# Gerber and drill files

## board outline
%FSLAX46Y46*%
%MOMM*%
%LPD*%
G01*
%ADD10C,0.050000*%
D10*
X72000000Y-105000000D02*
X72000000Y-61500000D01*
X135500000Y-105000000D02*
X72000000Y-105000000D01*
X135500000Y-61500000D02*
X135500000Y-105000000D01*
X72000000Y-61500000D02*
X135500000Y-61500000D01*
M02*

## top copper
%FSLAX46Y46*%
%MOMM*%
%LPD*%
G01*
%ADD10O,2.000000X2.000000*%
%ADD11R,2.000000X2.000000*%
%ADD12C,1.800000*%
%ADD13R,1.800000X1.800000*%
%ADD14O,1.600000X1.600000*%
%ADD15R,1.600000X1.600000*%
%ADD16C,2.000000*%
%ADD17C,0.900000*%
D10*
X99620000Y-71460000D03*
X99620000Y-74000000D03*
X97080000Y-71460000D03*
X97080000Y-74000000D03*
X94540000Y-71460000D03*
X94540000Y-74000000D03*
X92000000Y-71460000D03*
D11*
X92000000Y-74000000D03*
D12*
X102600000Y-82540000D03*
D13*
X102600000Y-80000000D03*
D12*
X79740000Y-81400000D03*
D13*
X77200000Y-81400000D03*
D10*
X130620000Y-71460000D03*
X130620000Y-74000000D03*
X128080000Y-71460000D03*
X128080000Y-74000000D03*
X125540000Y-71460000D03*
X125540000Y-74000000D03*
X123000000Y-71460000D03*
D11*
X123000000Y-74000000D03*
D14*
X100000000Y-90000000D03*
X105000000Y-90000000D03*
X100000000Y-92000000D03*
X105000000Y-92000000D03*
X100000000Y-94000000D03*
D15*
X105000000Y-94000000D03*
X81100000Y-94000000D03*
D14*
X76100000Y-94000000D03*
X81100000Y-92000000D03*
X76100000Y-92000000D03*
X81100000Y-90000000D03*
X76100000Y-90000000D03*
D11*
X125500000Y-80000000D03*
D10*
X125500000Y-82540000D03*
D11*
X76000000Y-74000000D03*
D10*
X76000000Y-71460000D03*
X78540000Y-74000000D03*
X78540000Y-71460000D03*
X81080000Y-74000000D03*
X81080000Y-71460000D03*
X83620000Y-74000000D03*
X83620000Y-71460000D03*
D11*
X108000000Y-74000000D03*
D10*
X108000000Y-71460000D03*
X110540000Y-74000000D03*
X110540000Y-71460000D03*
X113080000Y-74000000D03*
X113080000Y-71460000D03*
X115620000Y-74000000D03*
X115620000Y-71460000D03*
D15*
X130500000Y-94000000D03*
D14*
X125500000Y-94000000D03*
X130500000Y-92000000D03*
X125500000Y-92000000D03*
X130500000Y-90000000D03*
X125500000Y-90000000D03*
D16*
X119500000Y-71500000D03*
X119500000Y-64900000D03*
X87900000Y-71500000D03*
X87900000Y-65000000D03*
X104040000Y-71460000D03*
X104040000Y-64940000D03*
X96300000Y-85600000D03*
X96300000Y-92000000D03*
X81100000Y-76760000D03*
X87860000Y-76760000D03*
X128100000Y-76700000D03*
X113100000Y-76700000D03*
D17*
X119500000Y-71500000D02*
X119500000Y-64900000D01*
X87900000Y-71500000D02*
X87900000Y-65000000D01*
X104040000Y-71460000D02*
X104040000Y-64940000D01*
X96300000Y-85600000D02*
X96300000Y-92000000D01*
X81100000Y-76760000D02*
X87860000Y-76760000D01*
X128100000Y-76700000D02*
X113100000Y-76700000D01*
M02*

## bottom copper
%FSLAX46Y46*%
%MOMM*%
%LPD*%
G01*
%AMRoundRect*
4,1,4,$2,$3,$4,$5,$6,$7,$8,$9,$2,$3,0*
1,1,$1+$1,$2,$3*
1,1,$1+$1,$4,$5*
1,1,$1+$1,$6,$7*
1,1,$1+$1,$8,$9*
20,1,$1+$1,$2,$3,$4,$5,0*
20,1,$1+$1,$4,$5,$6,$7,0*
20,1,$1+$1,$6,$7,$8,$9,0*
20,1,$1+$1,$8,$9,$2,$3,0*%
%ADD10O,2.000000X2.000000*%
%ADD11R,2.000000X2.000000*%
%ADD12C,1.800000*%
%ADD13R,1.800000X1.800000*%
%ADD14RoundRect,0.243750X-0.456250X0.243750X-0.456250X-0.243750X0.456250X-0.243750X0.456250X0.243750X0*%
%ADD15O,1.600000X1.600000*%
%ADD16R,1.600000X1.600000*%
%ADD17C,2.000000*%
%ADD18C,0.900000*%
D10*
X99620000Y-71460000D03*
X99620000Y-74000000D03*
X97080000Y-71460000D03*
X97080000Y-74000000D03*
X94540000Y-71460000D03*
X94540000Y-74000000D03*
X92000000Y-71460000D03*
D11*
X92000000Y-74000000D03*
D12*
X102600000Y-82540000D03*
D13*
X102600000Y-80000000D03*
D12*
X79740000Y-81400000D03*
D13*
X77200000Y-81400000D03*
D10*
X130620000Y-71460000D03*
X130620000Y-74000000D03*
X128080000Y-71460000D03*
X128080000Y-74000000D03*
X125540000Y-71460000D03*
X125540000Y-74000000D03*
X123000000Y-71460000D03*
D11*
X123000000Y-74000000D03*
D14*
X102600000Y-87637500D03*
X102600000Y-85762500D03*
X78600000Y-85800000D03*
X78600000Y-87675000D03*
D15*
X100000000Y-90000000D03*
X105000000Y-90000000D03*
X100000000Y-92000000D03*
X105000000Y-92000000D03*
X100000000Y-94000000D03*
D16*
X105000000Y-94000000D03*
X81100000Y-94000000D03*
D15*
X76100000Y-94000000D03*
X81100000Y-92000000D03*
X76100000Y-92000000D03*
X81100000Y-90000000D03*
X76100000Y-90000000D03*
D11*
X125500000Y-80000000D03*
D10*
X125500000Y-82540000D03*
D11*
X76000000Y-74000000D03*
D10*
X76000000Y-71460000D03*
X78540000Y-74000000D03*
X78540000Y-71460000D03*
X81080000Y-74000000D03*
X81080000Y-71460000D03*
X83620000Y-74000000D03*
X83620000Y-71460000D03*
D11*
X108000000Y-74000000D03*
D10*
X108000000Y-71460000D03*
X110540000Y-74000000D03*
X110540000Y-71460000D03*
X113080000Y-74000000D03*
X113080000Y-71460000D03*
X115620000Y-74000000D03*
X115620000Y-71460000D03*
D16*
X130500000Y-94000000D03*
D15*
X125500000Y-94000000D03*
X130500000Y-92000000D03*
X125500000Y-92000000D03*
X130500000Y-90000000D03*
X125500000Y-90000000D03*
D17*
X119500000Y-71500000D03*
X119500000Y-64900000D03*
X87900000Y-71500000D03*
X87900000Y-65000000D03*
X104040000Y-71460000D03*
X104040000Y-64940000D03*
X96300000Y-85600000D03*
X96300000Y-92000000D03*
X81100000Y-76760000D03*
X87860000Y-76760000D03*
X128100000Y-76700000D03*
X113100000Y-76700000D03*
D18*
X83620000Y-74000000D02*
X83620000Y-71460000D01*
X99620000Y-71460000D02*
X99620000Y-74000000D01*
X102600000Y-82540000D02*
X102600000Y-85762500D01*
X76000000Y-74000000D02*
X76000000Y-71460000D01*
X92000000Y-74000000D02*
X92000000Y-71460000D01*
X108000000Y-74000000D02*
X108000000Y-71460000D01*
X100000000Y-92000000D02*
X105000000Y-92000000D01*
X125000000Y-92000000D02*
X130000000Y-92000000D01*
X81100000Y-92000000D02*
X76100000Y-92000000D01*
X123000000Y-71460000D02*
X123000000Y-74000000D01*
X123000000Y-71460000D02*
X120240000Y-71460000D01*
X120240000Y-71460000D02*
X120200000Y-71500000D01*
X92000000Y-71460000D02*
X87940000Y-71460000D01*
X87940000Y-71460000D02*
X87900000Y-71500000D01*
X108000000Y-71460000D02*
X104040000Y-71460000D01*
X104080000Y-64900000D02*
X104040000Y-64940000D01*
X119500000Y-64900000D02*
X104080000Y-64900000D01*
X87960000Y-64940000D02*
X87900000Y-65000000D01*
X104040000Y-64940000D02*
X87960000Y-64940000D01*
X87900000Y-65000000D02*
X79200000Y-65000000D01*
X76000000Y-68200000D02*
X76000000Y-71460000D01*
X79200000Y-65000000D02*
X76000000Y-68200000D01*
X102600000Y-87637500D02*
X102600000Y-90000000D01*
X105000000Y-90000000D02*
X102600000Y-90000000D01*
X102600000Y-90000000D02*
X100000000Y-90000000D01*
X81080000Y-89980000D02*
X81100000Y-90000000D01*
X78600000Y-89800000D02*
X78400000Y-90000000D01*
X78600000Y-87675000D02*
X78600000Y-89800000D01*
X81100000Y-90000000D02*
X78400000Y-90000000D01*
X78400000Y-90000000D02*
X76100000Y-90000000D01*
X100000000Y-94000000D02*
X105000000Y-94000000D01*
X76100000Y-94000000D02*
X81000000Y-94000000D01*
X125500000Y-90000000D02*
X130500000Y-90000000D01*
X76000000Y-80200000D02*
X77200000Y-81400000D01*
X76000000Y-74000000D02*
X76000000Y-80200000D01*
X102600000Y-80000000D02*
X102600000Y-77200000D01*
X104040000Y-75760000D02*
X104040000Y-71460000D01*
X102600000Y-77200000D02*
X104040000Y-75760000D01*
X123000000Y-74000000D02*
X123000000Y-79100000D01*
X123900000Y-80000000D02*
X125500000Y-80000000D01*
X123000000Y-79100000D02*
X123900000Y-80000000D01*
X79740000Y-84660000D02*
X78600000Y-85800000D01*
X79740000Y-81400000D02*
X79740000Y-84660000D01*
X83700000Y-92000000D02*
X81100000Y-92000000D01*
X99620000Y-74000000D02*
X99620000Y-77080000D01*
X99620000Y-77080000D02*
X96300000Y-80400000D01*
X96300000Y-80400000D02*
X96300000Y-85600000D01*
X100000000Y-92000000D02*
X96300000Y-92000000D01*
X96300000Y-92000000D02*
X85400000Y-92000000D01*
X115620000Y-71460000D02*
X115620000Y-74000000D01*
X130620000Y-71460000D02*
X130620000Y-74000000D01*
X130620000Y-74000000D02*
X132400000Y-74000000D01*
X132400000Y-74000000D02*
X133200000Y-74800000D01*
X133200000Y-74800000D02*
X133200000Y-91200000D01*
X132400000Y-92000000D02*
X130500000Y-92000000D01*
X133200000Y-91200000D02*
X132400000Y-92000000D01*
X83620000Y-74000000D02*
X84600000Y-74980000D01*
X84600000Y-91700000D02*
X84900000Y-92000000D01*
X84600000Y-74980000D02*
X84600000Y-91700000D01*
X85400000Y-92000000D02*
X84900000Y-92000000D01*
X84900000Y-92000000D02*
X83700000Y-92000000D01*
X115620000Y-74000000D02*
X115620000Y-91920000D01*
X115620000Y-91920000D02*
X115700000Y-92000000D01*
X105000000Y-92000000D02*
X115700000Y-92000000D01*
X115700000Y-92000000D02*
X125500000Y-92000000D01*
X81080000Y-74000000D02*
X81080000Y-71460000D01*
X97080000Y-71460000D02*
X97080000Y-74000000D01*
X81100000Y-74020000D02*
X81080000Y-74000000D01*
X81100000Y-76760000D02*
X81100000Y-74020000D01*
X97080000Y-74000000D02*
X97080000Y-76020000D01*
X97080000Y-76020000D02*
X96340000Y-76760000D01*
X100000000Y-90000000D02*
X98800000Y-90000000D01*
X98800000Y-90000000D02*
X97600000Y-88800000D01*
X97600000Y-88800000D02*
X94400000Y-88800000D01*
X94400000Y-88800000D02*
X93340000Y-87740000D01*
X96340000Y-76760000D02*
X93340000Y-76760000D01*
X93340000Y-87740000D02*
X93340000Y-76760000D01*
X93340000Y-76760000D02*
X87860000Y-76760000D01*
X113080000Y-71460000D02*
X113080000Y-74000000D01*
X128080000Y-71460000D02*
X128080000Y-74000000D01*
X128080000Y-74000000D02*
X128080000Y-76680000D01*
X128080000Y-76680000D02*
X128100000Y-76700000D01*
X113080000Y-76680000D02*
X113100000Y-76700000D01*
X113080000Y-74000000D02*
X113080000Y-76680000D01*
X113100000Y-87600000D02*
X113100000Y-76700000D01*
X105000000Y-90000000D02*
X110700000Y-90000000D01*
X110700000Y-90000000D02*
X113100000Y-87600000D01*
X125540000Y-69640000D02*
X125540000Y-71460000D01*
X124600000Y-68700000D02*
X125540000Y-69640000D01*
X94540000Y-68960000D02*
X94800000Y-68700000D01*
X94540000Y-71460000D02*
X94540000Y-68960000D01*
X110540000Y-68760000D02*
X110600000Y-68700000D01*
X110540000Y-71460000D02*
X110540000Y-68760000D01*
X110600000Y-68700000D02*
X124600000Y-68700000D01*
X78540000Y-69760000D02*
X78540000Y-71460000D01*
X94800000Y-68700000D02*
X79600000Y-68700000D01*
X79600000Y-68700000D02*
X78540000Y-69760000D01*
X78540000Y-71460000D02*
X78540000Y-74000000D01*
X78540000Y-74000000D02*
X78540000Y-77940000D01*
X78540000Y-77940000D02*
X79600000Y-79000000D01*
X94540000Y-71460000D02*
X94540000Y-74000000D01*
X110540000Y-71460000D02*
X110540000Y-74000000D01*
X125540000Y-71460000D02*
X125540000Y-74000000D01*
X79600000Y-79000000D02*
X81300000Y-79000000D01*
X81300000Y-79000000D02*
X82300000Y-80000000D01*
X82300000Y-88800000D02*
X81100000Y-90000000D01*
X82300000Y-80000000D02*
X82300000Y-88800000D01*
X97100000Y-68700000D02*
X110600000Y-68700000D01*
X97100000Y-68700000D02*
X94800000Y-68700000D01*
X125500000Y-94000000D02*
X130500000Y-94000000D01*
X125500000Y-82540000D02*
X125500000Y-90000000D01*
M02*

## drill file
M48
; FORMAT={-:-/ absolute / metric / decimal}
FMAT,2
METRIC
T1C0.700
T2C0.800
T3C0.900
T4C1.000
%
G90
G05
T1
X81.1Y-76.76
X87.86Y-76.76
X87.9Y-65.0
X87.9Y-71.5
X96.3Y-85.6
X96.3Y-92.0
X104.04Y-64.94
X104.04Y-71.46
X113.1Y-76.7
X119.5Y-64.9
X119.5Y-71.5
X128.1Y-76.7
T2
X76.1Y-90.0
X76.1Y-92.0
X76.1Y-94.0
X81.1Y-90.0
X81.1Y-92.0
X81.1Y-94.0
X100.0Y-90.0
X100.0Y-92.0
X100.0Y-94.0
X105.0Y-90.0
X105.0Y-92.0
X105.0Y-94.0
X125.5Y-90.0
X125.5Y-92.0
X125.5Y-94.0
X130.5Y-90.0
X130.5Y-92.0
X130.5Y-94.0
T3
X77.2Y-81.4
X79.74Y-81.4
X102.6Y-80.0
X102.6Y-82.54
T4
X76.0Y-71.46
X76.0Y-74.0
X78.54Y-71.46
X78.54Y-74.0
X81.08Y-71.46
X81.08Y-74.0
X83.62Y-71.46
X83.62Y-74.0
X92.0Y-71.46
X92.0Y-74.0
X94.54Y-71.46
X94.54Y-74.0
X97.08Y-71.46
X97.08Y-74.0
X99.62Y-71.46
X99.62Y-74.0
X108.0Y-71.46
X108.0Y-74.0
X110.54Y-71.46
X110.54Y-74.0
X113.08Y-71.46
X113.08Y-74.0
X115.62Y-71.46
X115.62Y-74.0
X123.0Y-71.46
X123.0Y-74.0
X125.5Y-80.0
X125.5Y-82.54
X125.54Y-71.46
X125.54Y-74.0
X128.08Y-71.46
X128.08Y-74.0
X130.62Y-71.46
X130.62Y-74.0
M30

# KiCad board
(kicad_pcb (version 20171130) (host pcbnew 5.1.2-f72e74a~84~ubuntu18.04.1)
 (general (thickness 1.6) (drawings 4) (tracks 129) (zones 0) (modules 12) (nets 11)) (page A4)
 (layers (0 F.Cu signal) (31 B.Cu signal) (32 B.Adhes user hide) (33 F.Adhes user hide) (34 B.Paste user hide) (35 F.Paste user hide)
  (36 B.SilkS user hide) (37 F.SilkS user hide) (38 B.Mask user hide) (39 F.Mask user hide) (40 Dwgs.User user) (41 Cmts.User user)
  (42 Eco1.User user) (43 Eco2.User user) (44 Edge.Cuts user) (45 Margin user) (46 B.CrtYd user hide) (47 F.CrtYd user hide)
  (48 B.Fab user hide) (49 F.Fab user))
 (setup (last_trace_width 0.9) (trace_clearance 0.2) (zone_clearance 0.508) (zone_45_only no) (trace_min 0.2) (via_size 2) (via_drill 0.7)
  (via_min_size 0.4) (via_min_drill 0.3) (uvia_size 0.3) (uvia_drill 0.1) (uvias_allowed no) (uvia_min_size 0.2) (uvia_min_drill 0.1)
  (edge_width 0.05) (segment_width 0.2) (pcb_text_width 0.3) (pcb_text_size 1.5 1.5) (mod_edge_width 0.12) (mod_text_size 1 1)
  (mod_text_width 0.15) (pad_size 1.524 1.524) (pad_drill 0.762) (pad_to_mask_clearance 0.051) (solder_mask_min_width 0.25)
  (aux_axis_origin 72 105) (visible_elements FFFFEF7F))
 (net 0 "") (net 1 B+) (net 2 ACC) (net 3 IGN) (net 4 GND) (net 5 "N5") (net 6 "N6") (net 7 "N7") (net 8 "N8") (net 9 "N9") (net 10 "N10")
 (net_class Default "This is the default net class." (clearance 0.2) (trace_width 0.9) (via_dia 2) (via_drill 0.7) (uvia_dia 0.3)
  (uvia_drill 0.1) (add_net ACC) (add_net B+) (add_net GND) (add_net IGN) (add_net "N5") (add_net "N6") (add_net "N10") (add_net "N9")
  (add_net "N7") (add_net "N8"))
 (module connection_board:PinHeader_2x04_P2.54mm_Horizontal (layer F.Cu) (at 92 74 90)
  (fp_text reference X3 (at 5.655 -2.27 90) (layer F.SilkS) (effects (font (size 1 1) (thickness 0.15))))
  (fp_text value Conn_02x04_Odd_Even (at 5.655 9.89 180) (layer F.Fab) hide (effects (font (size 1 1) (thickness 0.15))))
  (pad 8 thru_hole oval (at 2.54 7.62 90) (size 2 2) (drill 1) (layers *.Cu *.Mask) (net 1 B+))
  (pad 7 thru_hole oval (at 0 7.62 90) (size 2 2) (drill 1) (layers *.Cu *.Mask) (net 1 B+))
  (pad 6 thru_hole oval (at 2.54 5.08 90) (size 2 2) (drill 1) (layers *.Cu *.Mask) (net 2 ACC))
  (pad 5 thru_hole oval (at 0 5.08 90) (size 2 2) (drill 1) (layers *.Cu *.Mask) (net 2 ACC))
  (pad 4 thru_hole oval (at 2.54 2.54 90) (size 2 2) (drill 1) (layers *.Cu *.Mask) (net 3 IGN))
  (pad 3 thru_hole oval (at 0 2.54 90) (size 2 2) (drill 1) (layers *.Cu *.Mask) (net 3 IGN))
  (pad 2 thru_hole oval (at 2.54 0 90) (size 2 2) (drill 1) (layers *.Cu *.Mask) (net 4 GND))
  (pad 1 thru_hole rect (at 0 0 90) (size 2 2) (drill 1) (layers *.Cu *.Mask) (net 4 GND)))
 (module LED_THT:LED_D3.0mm (layer F.Cu) (at 102.6 80 270)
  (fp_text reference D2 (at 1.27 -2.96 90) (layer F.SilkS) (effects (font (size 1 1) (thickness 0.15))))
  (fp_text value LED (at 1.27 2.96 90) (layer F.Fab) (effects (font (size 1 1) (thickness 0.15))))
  (pad 2 thru_hole circle (at 2.54 0 270) (size 1.8 1.8) (drill 0.9) (layers *.Cu *.Mask) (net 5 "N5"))
  (pad 1 thru_hole rect (at 0 0 270) (size 1.8 1.8) (drill 0.9) (layers *.Cu *.Mask) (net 4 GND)))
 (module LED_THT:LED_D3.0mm (layer F.Cu) (at 77.2 81.4)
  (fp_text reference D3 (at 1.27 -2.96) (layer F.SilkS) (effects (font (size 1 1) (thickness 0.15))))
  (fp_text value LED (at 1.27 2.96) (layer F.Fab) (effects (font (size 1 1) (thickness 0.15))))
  (pad 2 thru_hole circle (at 2.54 0) (size 1.8 1.8) (drill 0.9) (layers *.Cu *.Mask) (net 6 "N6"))
  (pad 1 thru_hole rect (at 0 0) (size 1.8 1.8) (drill 0.9) (layers *.Cu *.Mask) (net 4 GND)))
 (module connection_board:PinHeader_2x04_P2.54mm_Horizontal (layer F.Cu) (at 123 74 90)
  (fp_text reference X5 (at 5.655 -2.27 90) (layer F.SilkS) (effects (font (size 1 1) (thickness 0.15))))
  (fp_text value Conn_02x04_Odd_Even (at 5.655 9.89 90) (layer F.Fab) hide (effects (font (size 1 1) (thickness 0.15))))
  (pad 8 thru_hole oval (at 2.54 7.62 90) (size 2 2) (drill 1) (layers *.Cu *.Mask) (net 1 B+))
  (pad 7 thru_hole oval (at 0 7.62 90) (size 2 2) (drill 1) (layers *.Cu *.Mask) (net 1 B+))
  (pad 6 thru_hole oval (at 2.54 5.08 90) (size 2 2) (drill 1) (layers *.Cu *.Mask) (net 2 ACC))
  (pad 5 thru_hole oval (at 0 5.08 90) (size 2 2) (drill 1) (layers *.Cu *.Mask) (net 2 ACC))
  (pad 4 thru_hole oval (at 2.54 2.54 90) (size 2 2) (drill 1) (layers *.Cu *.Mask) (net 3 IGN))
  (pad 3 thru_hole oval (at 0 2.54 90) (size 2 2) (drill 1) (layers *.Cu *.Mask) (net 3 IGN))
  (pad 2 thru_hole oval (at 2.54 0 90) (size 2 2) (drill 1) (layers *.Cu *.Mask) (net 4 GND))
  (pad 1 thru_hole rect (at 0 0 90) (size 2 2) (drill 1) (layers *.Cu *.Mask) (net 4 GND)))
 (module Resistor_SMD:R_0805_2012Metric (layer B.Cu) (at 102.6 86.7 270)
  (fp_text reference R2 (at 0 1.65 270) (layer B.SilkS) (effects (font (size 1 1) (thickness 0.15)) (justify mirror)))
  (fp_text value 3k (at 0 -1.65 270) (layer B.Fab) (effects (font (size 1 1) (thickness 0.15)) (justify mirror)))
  (pad 2 smd roundrect (at 0.9375 0 270) (size 0.975 1.4) (layers B.Cu B.Paste B.Mask) (roundrect_rratio 0.25) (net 2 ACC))
  (pad 1 smd roundrect (at -0.9375 0 270) (size 0.975 1.4) (layers B.Cu B.Paste B.Mask) (roundrect_rratio 0.25) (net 5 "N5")))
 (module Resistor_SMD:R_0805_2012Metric (layer B.Cu) (at 78.6 86.7375 270)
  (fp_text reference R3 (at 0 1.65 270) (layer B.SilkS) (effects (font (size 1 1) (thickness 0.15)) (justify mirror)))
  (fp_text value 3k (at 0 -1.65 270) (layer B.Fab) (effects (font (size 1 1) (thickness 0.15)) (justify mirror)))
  (pad 1 smd roundrect (at -0.9375 0 270) (size 0.975 1.4) (layers B.Cu B.Paste B.Mask) (roundrect_rratio 0.25) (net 6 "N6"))
  (pad 2 smd roundrect (at 0.9375 0 270) (size 0.975 1.4) (layers B.Cu B.Paste B.Mask) (roundrect_rratio 0.25) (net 3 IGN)))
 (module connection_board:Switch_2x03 (layer F.Cu) (at 105 94 180)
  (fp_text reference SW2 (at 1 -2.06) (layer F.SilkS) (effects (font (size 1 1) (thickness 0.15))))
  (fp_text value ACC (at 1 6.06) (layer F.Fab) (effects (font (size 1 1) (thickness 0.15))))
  (pad 6 thru_hole oval (at 5 4 180) (size 1.6 1.6) (drill 0.8) (layers *.Cu *.Mask) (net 2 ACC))
  (pad 3 thru_hole oval (at 0 4 180) (size 1.6 1.6) (drill 0.8) (layers *.Cu *.Mask) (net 2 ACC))
  (pad 5 thru_hole oval (at 5 2 180) (size 1.6 1.6) (drill 0.8) (layers *.Cu *.Mask) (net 1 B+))
  (pad 2 thru_hole oval (at 0 2 180) (size 1.6 1.6) (drill 0.8) (layers *.Cu *.Mask) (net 1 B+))
  (pad 4 thru_hole oval (at 5 0 180) (size 1.6 1.6) (drill 0.8) (layers *.Cu *.Mask) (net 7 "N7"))
  (pad 1 thru_hole rect (at 0 0 180) (size 1.6 1.6) (drill 0.8) (layers *.Cu *.Mask) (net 7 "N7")))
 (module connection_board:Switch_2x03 (layer F.Cu) (at 81.1 94 180)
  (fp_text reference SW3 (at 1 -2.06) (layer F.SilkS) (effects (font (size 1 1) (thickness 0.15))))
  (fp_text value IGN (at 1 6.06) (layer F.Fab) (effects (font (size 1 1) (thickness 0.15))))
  (pad 1 thru_hole rect (at 0 0 180) (size 1.6 1.6) (drill 0.8) (layers *.Cu *.Mask) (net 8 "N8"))
  (pad 4 thru_hole oval (at 5 0 180) (size 1.6 1.6) (drill 0.8) (layers *.Cu *.Mask) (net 8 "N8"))
  (pad 2 thru_hole oval (at 0 2 180) (size 1.6 1.6) (drill 0.8) (layers *.Cu *.Mask) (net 1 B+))
  (pad 5 thru_hole oval (at 5 2 180) (size 1.6 1.6) (drill 0.8) (layers *.Cu *.Mask) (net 1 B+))
  (pad 3 thru_hole oval (at 0 4 180) (size 1.6 1.6) (drill 0.8) (layers *.Cu *.Mask) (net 3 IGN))
  (pad 6 thru_hole oval (at 5 4 180) (size 1.6 1.6) (drill 0.8) (layers *.Cu *.Mask) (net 3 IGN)))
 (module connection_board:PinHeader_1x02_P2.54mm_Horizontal (layer F.Cu) (at 125.5 80)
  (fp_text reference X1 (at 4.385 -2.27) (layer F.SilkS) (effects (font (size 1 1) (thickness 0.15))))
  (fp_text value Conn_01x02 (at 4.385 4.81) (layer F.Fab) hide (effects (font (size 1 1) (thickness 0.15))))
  (pad 1 thru_hole rect (at 0 0) (size 2 2) (drill 1) (layers *.Cu *.Mask) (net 4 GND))
  (pad 2 thru_hole oval (at 0 2.54) (size 2 2) (drill 1) (layers *.Cu *.Mask) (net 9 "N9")))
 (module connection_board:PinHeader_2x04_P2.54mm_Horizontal (layer F.Cu) (at 76 74 90)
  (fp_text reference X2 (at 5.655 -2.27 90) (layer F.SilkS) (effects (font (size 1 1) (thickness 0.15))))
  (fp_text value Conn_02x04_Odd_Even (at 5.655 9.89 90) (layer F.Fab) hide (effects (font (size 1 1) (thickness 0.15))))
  (pad 1 thru_hole rect (at 0 0 90) (size 2 2) (drill 1) (layers *.Cu *.Mask) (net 4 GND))
  (pad 2 thru_hole oval (at 2.54 0 90) (size 2 2) (drill 1) (layers *.Cu *.Mask) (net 4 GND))
  (pad 3 thru_hole oval (at 0 2.54 90) (size 2 2) (drill 1) (layers *.Cu *.Mask) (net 3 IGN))
  (pad 4 thru_hole oval (at 2.54 2.54 90) (size 2 2) (drill 1) (layers *.Cu *.Mask) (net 3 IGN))
  (pad 5 thru_hole oval (at 0 5.08 90) (size 2 2) (drill 1) (layers *.Cu *.Mask) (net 2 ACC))
  (pad 6 thru_hole oval (at 2.54 5.08 90) (size 2 2) (drill 1) (layers *.Cu *.Mask) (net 2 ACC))
  (pad 7 thru_hole oval (at 0 7.62 90) (size 2 2) (drill 1) (layers *.Cu *.Mask) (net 1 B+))
  (pad 8 thru_hole oval (at 2.54 7.62 90) (size 2 2) (drill 1) (layers *.Cu *.Mask) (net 1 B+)))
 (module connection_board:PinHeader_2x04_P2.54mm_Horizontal (layer F.Cu) (at 108 74 90)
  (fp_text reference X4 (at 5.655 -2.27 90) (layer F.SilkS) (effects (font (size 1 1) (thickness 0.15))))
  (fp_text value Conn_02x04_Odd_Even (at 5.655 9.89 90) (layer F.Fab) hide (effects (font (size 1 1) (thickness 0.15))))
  (pad 1 thru_hole rect (at 0 0 90) (size 2 2) (drill 1) (layers *.Cu *.Mask) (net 4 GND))
  (pad 2 thru_hole oval (at 2.54 0 90) (size 2 2) (drill 1) (layers *.Cu *.Mask) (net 4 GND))
  (pad 3 thru_hole oval (at 0 2.54 90) (size 2 2) (drill 1) (layers *.Cu *.Mask) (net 3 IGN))
  (pad 4 thru_hole oval (at 2.54 2.54 90) (size 2 2) (drill 1) (layers *.Cu *.Mask) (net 3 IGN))
  (pad 5 thru_hole oval (at 0 5.08 90) (size 2 2) (drill 1) (layers *.Cu *.Mask) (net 2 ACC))
  (pad 6 thru_hole oval (at 2.54 5.08 90) (size 2 2) (drill 1) (layers *.Cu *.Mask) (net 2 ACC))
  (pad 7 thru_hole oval (at 0 7.62 90) (size 2 2) (drill 1) (layers *.Cu *.Mask) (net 1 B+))
  (pad 8 thru_hole oval (at 2.54 7.62 90) (size 2 2) (drill 1) (layers *.Cu *.Mask) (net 1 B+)))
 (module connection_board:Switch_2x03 (layer F.Cu) (at 130.5 94 180)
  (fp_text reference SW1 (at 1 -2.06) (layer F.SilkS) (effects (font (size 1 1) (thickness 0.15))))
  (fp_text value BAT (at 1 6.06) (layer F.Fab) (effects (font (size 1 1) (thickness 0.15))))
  (pad 1 thru_hole rect (at 0 0 180) (size 1.6 1.6) (drill 0.8) (layers *.Cu *.Mask) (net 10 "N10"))
  (pad 4 thru_hole oval (at 5 0 180) (size 1.6 1.6) (drill 0.8) (layers *.Cu *.Mask) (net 10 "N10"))
  (pad 2 thru_hole oval (at 0 2 180) (size 1.6 1.6) (drill 0.8) (layers *.Cu *.Mask) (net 1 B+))
  (pad 5 thru_hole oval (at 5 2 180) (size 1.6 1.6) (drill 0.8) (layers *.Cu *.Mask) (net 1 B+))
  (pad 3 thru_hole oval (at 0 4 180) (size 1.6 1.6) (drill 0.8) (layers *.Cu *.Mask) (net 9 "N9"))
  (pad 6 thru_hole oval (at 5 4 180) (size 1.6 1.6) (drill 0.8) (layers *.Cu *.Mask) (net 9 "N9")))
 (gr_line (start 72 105) (end 72 61.5) (layer Edge.Cuts) (width 0.05))
 (gr_line (start 135.5 105) (end 72 105) (layer Edge.Cuts) (width 0.05))
 (gr_line (start 135.5 61.5) (end 135.5 105) (layer Edge.Cuts) (width 0.05))
 (gr_line (start 72 61.5) (end 135.5 61.5) (layer Edge.Cuts) (width 0.05))
 (segment (start 83.62 74) (end 83.62 71.46) (width 0.9) (layer B.Cu) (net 1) (status 30))
 (segment (start 99.62 71.46) (end 99.62 74) (width 0.9) (layer B.Cu) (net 1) (status 30))
 (segment (start 102.6 82.54) (end 102.6 85.7625) (width 0.9) (layer B.Cu) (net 5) (status 30))
 (segment (start 76 74) (end 76 71.46) (width 0.9) (layer B.Cu) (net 4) (status 30))
 (segment (start 92 74) (end 92 71.46) (width 0.9) (layer B.Cu) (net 4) (status 30))
 (segment (start 108 74) (end 108 71.46) (width 0.9) (layer B.Cu) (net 4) (status 30))
 (segment (start 100 92) (end 105 92) (width 0.9) (layer B.Cu) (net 1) (status 30))
 (segment (start 125 92) (end 130 92) (width 0.9) (layer B.Cu) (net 1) (status 30))
 (segment (start 81.1 92) (end 76.1 92) (width 0.9) (layer B.Cu) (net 1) (status 30))
 (segment (start 123 71.46) (end 123 74) (width 0.9) (layer B.Cu) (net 4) (status 30))
 (via (at 119.5 71.5) (size 2) (drill 0.7) (layers F.Cu B.Cu) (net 4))
 (segment (start 123 71.46) (end 120.24 71.46) (width 0.9) (layer B.Cu) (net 4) (status 10))
 (segment (start 120.24 71.46) (end 120.2 71.5) (width 0.9) (layer B.Cu) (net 4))
 (segment (start 119.5 71.5) (end 119.5 64.9) (width 0.9) (layer F.Cu) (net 4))
 (via (at 119.5 64.9) (size 2) (drill 0.7) (layers F.Cu B.Cu) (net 4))
 (via (at 87.9 71.5) (size 2) (drill 0.7) (layers F.Cu B.Cu) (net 4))
 (segment (start 92 71.46) (end 87.94 71.46) (width 0.9) (layer B.Cu) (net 4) (status 10))
 (segment (start 87.94 71.46) (end 87.9 71.5) (width 0.9) (layer B.Cu) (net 4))
 (segment (start 87.9 71.5) (end 87.9 65) (width 0.9) (layer F.Cu) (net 4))
 (via (at 87.9 65) (size 2) (drill 0.7) (layers F.Cu B.Cu) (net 4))
 (segment (start 108 71.46) (end 104.04 71.46) (width 0.9) (layer B.Cu) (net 4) (status 10))
 (via (at 104.04 71.46) (size 2) (drill 0.7) (layers F.Cu B.Cu) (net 4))
 (segment (start 104.04 71.46) (end 104.04 64.94) (width 0.9) (layer F.Cu) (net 4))
 (via (at 104.04 64.94) (size 2) (drill 0.7) (layers F.Cu B.Cu) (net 4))
 (segment (start 104.08 64.9) (end 104.04 64.94) (width 0.9) (layer B.Cu) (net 4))
 (segment (start 119.5 64.9) (end 104.08 64.9) (width 0.9) (layer B.Cu) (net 4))
 (segment (start 87.96 64.94) (end 87.9 65) (width 0.9) (layer B.Cu) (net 4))
 (segment (start 104.04 64.94) (end 87.96 64.94) (width 0.9) (layer B.Cu) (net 4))
 (segment (start 87.9 65) (end 79.2 65) (width 0.9) (layer B.Cu) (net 4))
 (segment (start 76 68.2) (end 76 71.46) (width 0.9) (layer B.Cu) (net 4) (status 20))
 (segment (start 79.2 65) (end 76 68.2) (width 0.9) (layer B.Cu) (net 4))
 (segment (start 102.6 87.6375) (end 102.6 90) (width 0.9) (layer B.Cu) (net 2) (status 10))
 (segment (start 105 90) (end 102.6 90) (width 0.9) (layer B.Cu) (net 2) (status 10))
 (segment (start 102.6 90) (end 100 90) (width 0.9) (layer B.Cu) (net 2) (status 20))
 (segment (start 81.08 89.98) (end 81.1 90) (width 0.9) (layer B.Cu) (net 3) (status 30))
 (segment (start 78.6 89.8) (end 78.4 90) (width 0.9) (layer B.Cu) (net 3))
 (segment (start 78.6 87.675) (end 78.6 89.8) (width 0.9) (layer B.Cu) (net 3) (status 10))
 (segment (start 81.1 90) (end 78.4 90) (width 0.9) (layer B.Cu) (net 3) (status 10))
 (segment (start 78.4 90) (end 76.1 90) (width 0.9) (layer B.Cu) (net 3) (status 20))
 (segment (start 100 94) (end 105 94) (width 0.9) (layer B.Cu) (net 7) (status 30))
 (segment (start 76.1 94) (end 81 94) (width 0.9) (layer B.Cu) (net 8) (status 30))
 (segment (start 125.5 90) (end 130.5 90) (width 0.9) (layer B.Cu) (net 9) (status 30))
 (segment (start 76 80.2) (end 77.2 81.4) (width 0.9) (layer B.Cu) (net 4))
 (segment (start 76 74) (end 76 80.2) (width 0.9) (layer B.Cu) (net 4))
 (segment (start 102.6 80) (end 102.6 77.2) (width 0.9) (layer B.Cu) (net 4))
 (segment (start 104.04 75.76) (end 104.04 71.46) (width 0.9) (layer B.Cu) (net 4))
 (segment (start 102.6 77.2) (end 104.04 75.76) (width 0.9) (layer B.Cu) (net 4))
 (segment (start 123 74) (end 123 79.1) (width 0.9) (layer B.Cu) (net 4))
 (segment (start 123.9 80) (end 125.5 80) (width 0.9) (layer B.Cu) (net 4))
 (segment (start 123 79.1) (end 123.9 80) (width 0.9) (layer B.Cu) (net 4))
 (segment (start 79.74 84.66) (end 78.6 85.8) (width 0.9) (layer B.Cu) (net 6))
 (segment (start 79.74 81.4) (end 79.74 84.66) (width 0.9) (layer B.Cu) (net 6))
 (segment (start 83.7 92) (end 81.1 92) (width 0.9) (layer B.Cu) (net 1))
 (segment (start 99.62 74) (end 99.62 77.08) (width 0.9) (layer B.Cu) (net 1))
 (segment (start 99.62 77.08) (end 96.3 80.4) (width 0.9) (layer B.Cu) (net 1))
 (via (at 96.3 85.6) (size 2) (drill 0.7) (layers F.Cu B.Cu) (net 1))
 (segment (start 96.3 80.4) (end 96.3 85.6) (width 0.9) (layer B.Cu) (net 1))
 (via (at 96.3 92) (size 2) (drill 0.7) (layers F.Cu B.Cu) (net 1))
 (segment (start 96.3 85.6) (end 96.3 92) (width 0.9) (layer F.Cu) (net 1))
 (segment (start 100 92) (end 96.3 92) (width 0.9) (layer B.Cu) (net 1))
 (segment (start 96.3 92) (end 85.4 92) (width 0.9) (layer B.Cu) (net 1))
 (segment (start 115.62 71.46) (end 115.62 74) (width 0.9) (layer B.Cu) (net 1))
 (segment (start 130.62 71.46) (end 130.62 74) (width 0.9) (layer B.Cu) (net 1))
 (segment (start 130.62 74) (end 132.4 74) (width 0.9) (layer B.Cu) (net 1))
 (segment (start 132.4 74) (end 133.2 74.8) (width 0.9) (layer B.Cu) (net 1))
 (segment (start 133.2 74.8) (end 133.2 91.2) (width 0.9) (layer B.Cu) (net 1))
 (segment (start 132.4 92) (end 130.5 92) (width 0.9) (layer B.Cu) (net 1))
 (segment (start 133.2 91.2) (end 132.4 92) (width 0.9) (layer B.Cu) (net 1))
 (segment (start 83.62 74) (end 84.6 74.98) (width 0.9) (layer B.Cu) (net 1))
 (segment (start 84.6 91.7) (end 84.9 92) (width 0.9) (layer B.Cu) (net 1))
 (segment (start 84.6 74.98) (end 84.6 91.7) (width 0.9) (layer B.Cu) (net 1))
 (segment (start 85.4 92) (end 84.9 92) (width 0.9) (layer B.Cu) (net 1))
 (segment (start 84.9 92) (end 83.7 92) (width 0.9) (layer B.Cu) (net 1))
 (segment (start 115.62 74) (end 115.62 91.92) (width 0.9) (layer B.Cu) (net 1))
 (segment (start 115.62 91.92) (end 115.7 92) (width 0.9) (layer B.Cu) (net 1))
 (segment (start 105 92) (end 115.7 92) (width 0.9) (layer B.Cu) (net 1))
 (segment (start 115.7 92) (end 125.5 92) (width 0.9) (layer B.Cu) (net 1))
 (segment (start 81.08 74) (end 81.08 71.46) (width 0.9) (layer B.Cu) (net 2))
 (segment (start 97.08 71.46) (end 97.08 74) (width 0.9) (layer B.Cu) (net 2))
 (via (at 81.1 76.76) (size 2) (drill 0.7) (layers F.Cu B.Cu) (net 2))
 (via (at 87.86 76.76) (size 2) (drill 0.7) (layers F.Cu B.Cu) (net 2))
 (segment (start 81.1 74.02) (end 81.08 74) (width 0.9) (layer B.Cu) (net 2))
 (segment (start 81.1 76.76) (end 87.86 76.76) (width 0.9) (layer F.Cu) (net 2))
 (segment (start 81.1 76.76) (end 81.1 74.02) (width 0.9) (layer B.Cu) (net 2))
 (segment (start 97.08 74) (end 97.08 76.02) (width 0.9) (layer B.Cu) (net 2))
 (segment (start 97.08 76.02) (end 96.34 76.76) (width 0.9) (layer B.Cu) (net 2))
 (segment (start 100 90) (end 98.8 90) (width 0.9) (layer B.Cu) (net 2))
 (segment (start 98.8 90) (end 97.6 88.8) (width 0.9) (layer B.Cu) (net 2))
 (segment (start 97.6 88.8) (end 94.4 88.8) (width 0.9) (layer B.Cu) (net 2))
 (segment (start 94.4 88.8) (end 93.34 87.74) (width 0.9) (layer B.Cu) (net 2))
 (segment (start 96.34 76.76) (end 93.34 76.76) (width 0.9) (layer B.Cu) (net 2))
 (segment (start 93.34 87.74) (end 93.34 76.76) (width 0.9) (layer B.Cu) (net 2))
 (segment (start 93.34 76.76) (end 87.86 76.76) (width 0.9) (layer B.Cu) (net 2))
 (segment (start 113.08 71.46) (end 113.08 74) (width 0.9) (layer B.Cu) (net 2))
 (segment (start 128.08 71.46) (end 128.08 74) (width 0.9) (layer B.Cu) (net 2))
 (segment (start 128.08 74) (end 128.08 76.68) (width 0.9) (layer B.Cu) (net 2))
 (via (at 128.1 76.7) (size 2) (drill 0.7) (layers F.Cu B.Cu) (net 2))
 (segment (start 128.08 76.68) (end 128.1 76.7) (width 0.9) (layer B.Cu) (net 2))
 (segment (start 128.1 76.7) (end 113.1 76.7) (width 0.9) (layer F.Cu) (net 2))
 (via (at 113.1 76.7) (size 2) (drill 0.7) (layers F.Cu B.Cu) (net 2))
 (segment (start 113.08 76.68) (end 113.1 76.7) (width 0.9) (layer B.Cu) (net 2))
 (segment (start 113.08 74) (end 113.08 76.68) (width 0.9) (layer B.Cu) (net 2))
 (segment (start 113.1 87.6) (end 113.1 76.7) (width 0.9) (layer B.Cu) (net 2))
 (segment (start 105 90) (end 110.7 90) (width 0.9) (layer B.Cu) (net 2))
 (segment (start 110.7 90) (end 113.1 87.6) (width 0.9) (layer B.Cu) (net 2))
 (segment (start 125.54 69.64) (end 125.54 71.46) (width 0.9) (layer B.Cu) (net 3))
 (segment (start 124.6 68.7) (end 125.54 69.64) (width 0.9) (layer B.Cu) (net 3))
 (segment (start 94.54 68.96) (end 94.8 68.7) (width 0.9) (layer B.Cu) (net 3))
 (segment (start 94.54 71.46) (end 94.54 68.96) (width 0.9) (layer B.Cu) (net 3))
 (segment (start 110.54 68.76) (end 110.6 68.7) (width 0.9) (layer B.Cu) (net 3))
 (segment (start 110.54 71.46) (end 110.54 68.76) (width 0.9) (layer B.Cu) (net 3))
 (segment (start 110.6 68.7) (end 124.6 68.7) (width 0.9) (layer B.Cu) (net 3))
 (segment (start 78.54 69.76) (end 78.54 71.46) (width 0.9) (layer B.Cu) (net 3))
 (segment (start 94.8 68.7) (end 79.6 68.7) (width 0.9) (layer B.Cu) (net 3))
 (segment (start 79.6 68.7) (end 78.54 69.76) (width 0.9) (layer B.Cu) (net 3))
 (segment (start 78.54 71.46) (end 78.54 74) (width 0.9) (layer B.Cu) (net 3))
 (segment (start 78.54 74) (end 78.54 77.94) (width 0.9) (layer B.Cu) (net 3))
 (segment (start 78.54 77.94) (end 79.6 79) (width 0.9) (layer B.Cu) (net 3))
 (segment (start 94.54 71.46) (end 94.54 74) (width 0.9) (layer B.Cu) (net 3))
 (segment (start 110.54 71.46) (end 110.54 74) (width 0.9) (layer B.Cu) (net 3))
 (segment (start 125.54 71.46) (end 125.54 74) (width 0.9) (layer B.Cu) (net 3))
 (segment (start 79.6 79) (end 81.3 79) (width 0.9) (layer B.Cu) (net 3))
 (segment (start 81.3 79) (end 82.3 80) (width 0.9) (layer B.Cu) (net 3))
 (segment (start 82.3 88.8) (end 81.1 90) (width 0.9) (layer B.Cu) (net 3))
 (segment (start 82.3 80) (end 82.3 88.8) (width 0.9) (layer B.Cu) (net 3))
 (segment (start 97.1 68.7) (end 110.6 68.7) (width 0.9) (layer B.Cu) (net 3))
 (segment (start 97.1 68.7) (end 94.8 68.7) (width 0.9) (layer B.Cu) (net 3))
 (segment (start 125.5 94) (end 130.5 94) (width 0.9) (layer B.Cu) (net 10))
 (segment (start 125.5 82.54) (end 125.5 90) (width 0.9) (layer B.Cu) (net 9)))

